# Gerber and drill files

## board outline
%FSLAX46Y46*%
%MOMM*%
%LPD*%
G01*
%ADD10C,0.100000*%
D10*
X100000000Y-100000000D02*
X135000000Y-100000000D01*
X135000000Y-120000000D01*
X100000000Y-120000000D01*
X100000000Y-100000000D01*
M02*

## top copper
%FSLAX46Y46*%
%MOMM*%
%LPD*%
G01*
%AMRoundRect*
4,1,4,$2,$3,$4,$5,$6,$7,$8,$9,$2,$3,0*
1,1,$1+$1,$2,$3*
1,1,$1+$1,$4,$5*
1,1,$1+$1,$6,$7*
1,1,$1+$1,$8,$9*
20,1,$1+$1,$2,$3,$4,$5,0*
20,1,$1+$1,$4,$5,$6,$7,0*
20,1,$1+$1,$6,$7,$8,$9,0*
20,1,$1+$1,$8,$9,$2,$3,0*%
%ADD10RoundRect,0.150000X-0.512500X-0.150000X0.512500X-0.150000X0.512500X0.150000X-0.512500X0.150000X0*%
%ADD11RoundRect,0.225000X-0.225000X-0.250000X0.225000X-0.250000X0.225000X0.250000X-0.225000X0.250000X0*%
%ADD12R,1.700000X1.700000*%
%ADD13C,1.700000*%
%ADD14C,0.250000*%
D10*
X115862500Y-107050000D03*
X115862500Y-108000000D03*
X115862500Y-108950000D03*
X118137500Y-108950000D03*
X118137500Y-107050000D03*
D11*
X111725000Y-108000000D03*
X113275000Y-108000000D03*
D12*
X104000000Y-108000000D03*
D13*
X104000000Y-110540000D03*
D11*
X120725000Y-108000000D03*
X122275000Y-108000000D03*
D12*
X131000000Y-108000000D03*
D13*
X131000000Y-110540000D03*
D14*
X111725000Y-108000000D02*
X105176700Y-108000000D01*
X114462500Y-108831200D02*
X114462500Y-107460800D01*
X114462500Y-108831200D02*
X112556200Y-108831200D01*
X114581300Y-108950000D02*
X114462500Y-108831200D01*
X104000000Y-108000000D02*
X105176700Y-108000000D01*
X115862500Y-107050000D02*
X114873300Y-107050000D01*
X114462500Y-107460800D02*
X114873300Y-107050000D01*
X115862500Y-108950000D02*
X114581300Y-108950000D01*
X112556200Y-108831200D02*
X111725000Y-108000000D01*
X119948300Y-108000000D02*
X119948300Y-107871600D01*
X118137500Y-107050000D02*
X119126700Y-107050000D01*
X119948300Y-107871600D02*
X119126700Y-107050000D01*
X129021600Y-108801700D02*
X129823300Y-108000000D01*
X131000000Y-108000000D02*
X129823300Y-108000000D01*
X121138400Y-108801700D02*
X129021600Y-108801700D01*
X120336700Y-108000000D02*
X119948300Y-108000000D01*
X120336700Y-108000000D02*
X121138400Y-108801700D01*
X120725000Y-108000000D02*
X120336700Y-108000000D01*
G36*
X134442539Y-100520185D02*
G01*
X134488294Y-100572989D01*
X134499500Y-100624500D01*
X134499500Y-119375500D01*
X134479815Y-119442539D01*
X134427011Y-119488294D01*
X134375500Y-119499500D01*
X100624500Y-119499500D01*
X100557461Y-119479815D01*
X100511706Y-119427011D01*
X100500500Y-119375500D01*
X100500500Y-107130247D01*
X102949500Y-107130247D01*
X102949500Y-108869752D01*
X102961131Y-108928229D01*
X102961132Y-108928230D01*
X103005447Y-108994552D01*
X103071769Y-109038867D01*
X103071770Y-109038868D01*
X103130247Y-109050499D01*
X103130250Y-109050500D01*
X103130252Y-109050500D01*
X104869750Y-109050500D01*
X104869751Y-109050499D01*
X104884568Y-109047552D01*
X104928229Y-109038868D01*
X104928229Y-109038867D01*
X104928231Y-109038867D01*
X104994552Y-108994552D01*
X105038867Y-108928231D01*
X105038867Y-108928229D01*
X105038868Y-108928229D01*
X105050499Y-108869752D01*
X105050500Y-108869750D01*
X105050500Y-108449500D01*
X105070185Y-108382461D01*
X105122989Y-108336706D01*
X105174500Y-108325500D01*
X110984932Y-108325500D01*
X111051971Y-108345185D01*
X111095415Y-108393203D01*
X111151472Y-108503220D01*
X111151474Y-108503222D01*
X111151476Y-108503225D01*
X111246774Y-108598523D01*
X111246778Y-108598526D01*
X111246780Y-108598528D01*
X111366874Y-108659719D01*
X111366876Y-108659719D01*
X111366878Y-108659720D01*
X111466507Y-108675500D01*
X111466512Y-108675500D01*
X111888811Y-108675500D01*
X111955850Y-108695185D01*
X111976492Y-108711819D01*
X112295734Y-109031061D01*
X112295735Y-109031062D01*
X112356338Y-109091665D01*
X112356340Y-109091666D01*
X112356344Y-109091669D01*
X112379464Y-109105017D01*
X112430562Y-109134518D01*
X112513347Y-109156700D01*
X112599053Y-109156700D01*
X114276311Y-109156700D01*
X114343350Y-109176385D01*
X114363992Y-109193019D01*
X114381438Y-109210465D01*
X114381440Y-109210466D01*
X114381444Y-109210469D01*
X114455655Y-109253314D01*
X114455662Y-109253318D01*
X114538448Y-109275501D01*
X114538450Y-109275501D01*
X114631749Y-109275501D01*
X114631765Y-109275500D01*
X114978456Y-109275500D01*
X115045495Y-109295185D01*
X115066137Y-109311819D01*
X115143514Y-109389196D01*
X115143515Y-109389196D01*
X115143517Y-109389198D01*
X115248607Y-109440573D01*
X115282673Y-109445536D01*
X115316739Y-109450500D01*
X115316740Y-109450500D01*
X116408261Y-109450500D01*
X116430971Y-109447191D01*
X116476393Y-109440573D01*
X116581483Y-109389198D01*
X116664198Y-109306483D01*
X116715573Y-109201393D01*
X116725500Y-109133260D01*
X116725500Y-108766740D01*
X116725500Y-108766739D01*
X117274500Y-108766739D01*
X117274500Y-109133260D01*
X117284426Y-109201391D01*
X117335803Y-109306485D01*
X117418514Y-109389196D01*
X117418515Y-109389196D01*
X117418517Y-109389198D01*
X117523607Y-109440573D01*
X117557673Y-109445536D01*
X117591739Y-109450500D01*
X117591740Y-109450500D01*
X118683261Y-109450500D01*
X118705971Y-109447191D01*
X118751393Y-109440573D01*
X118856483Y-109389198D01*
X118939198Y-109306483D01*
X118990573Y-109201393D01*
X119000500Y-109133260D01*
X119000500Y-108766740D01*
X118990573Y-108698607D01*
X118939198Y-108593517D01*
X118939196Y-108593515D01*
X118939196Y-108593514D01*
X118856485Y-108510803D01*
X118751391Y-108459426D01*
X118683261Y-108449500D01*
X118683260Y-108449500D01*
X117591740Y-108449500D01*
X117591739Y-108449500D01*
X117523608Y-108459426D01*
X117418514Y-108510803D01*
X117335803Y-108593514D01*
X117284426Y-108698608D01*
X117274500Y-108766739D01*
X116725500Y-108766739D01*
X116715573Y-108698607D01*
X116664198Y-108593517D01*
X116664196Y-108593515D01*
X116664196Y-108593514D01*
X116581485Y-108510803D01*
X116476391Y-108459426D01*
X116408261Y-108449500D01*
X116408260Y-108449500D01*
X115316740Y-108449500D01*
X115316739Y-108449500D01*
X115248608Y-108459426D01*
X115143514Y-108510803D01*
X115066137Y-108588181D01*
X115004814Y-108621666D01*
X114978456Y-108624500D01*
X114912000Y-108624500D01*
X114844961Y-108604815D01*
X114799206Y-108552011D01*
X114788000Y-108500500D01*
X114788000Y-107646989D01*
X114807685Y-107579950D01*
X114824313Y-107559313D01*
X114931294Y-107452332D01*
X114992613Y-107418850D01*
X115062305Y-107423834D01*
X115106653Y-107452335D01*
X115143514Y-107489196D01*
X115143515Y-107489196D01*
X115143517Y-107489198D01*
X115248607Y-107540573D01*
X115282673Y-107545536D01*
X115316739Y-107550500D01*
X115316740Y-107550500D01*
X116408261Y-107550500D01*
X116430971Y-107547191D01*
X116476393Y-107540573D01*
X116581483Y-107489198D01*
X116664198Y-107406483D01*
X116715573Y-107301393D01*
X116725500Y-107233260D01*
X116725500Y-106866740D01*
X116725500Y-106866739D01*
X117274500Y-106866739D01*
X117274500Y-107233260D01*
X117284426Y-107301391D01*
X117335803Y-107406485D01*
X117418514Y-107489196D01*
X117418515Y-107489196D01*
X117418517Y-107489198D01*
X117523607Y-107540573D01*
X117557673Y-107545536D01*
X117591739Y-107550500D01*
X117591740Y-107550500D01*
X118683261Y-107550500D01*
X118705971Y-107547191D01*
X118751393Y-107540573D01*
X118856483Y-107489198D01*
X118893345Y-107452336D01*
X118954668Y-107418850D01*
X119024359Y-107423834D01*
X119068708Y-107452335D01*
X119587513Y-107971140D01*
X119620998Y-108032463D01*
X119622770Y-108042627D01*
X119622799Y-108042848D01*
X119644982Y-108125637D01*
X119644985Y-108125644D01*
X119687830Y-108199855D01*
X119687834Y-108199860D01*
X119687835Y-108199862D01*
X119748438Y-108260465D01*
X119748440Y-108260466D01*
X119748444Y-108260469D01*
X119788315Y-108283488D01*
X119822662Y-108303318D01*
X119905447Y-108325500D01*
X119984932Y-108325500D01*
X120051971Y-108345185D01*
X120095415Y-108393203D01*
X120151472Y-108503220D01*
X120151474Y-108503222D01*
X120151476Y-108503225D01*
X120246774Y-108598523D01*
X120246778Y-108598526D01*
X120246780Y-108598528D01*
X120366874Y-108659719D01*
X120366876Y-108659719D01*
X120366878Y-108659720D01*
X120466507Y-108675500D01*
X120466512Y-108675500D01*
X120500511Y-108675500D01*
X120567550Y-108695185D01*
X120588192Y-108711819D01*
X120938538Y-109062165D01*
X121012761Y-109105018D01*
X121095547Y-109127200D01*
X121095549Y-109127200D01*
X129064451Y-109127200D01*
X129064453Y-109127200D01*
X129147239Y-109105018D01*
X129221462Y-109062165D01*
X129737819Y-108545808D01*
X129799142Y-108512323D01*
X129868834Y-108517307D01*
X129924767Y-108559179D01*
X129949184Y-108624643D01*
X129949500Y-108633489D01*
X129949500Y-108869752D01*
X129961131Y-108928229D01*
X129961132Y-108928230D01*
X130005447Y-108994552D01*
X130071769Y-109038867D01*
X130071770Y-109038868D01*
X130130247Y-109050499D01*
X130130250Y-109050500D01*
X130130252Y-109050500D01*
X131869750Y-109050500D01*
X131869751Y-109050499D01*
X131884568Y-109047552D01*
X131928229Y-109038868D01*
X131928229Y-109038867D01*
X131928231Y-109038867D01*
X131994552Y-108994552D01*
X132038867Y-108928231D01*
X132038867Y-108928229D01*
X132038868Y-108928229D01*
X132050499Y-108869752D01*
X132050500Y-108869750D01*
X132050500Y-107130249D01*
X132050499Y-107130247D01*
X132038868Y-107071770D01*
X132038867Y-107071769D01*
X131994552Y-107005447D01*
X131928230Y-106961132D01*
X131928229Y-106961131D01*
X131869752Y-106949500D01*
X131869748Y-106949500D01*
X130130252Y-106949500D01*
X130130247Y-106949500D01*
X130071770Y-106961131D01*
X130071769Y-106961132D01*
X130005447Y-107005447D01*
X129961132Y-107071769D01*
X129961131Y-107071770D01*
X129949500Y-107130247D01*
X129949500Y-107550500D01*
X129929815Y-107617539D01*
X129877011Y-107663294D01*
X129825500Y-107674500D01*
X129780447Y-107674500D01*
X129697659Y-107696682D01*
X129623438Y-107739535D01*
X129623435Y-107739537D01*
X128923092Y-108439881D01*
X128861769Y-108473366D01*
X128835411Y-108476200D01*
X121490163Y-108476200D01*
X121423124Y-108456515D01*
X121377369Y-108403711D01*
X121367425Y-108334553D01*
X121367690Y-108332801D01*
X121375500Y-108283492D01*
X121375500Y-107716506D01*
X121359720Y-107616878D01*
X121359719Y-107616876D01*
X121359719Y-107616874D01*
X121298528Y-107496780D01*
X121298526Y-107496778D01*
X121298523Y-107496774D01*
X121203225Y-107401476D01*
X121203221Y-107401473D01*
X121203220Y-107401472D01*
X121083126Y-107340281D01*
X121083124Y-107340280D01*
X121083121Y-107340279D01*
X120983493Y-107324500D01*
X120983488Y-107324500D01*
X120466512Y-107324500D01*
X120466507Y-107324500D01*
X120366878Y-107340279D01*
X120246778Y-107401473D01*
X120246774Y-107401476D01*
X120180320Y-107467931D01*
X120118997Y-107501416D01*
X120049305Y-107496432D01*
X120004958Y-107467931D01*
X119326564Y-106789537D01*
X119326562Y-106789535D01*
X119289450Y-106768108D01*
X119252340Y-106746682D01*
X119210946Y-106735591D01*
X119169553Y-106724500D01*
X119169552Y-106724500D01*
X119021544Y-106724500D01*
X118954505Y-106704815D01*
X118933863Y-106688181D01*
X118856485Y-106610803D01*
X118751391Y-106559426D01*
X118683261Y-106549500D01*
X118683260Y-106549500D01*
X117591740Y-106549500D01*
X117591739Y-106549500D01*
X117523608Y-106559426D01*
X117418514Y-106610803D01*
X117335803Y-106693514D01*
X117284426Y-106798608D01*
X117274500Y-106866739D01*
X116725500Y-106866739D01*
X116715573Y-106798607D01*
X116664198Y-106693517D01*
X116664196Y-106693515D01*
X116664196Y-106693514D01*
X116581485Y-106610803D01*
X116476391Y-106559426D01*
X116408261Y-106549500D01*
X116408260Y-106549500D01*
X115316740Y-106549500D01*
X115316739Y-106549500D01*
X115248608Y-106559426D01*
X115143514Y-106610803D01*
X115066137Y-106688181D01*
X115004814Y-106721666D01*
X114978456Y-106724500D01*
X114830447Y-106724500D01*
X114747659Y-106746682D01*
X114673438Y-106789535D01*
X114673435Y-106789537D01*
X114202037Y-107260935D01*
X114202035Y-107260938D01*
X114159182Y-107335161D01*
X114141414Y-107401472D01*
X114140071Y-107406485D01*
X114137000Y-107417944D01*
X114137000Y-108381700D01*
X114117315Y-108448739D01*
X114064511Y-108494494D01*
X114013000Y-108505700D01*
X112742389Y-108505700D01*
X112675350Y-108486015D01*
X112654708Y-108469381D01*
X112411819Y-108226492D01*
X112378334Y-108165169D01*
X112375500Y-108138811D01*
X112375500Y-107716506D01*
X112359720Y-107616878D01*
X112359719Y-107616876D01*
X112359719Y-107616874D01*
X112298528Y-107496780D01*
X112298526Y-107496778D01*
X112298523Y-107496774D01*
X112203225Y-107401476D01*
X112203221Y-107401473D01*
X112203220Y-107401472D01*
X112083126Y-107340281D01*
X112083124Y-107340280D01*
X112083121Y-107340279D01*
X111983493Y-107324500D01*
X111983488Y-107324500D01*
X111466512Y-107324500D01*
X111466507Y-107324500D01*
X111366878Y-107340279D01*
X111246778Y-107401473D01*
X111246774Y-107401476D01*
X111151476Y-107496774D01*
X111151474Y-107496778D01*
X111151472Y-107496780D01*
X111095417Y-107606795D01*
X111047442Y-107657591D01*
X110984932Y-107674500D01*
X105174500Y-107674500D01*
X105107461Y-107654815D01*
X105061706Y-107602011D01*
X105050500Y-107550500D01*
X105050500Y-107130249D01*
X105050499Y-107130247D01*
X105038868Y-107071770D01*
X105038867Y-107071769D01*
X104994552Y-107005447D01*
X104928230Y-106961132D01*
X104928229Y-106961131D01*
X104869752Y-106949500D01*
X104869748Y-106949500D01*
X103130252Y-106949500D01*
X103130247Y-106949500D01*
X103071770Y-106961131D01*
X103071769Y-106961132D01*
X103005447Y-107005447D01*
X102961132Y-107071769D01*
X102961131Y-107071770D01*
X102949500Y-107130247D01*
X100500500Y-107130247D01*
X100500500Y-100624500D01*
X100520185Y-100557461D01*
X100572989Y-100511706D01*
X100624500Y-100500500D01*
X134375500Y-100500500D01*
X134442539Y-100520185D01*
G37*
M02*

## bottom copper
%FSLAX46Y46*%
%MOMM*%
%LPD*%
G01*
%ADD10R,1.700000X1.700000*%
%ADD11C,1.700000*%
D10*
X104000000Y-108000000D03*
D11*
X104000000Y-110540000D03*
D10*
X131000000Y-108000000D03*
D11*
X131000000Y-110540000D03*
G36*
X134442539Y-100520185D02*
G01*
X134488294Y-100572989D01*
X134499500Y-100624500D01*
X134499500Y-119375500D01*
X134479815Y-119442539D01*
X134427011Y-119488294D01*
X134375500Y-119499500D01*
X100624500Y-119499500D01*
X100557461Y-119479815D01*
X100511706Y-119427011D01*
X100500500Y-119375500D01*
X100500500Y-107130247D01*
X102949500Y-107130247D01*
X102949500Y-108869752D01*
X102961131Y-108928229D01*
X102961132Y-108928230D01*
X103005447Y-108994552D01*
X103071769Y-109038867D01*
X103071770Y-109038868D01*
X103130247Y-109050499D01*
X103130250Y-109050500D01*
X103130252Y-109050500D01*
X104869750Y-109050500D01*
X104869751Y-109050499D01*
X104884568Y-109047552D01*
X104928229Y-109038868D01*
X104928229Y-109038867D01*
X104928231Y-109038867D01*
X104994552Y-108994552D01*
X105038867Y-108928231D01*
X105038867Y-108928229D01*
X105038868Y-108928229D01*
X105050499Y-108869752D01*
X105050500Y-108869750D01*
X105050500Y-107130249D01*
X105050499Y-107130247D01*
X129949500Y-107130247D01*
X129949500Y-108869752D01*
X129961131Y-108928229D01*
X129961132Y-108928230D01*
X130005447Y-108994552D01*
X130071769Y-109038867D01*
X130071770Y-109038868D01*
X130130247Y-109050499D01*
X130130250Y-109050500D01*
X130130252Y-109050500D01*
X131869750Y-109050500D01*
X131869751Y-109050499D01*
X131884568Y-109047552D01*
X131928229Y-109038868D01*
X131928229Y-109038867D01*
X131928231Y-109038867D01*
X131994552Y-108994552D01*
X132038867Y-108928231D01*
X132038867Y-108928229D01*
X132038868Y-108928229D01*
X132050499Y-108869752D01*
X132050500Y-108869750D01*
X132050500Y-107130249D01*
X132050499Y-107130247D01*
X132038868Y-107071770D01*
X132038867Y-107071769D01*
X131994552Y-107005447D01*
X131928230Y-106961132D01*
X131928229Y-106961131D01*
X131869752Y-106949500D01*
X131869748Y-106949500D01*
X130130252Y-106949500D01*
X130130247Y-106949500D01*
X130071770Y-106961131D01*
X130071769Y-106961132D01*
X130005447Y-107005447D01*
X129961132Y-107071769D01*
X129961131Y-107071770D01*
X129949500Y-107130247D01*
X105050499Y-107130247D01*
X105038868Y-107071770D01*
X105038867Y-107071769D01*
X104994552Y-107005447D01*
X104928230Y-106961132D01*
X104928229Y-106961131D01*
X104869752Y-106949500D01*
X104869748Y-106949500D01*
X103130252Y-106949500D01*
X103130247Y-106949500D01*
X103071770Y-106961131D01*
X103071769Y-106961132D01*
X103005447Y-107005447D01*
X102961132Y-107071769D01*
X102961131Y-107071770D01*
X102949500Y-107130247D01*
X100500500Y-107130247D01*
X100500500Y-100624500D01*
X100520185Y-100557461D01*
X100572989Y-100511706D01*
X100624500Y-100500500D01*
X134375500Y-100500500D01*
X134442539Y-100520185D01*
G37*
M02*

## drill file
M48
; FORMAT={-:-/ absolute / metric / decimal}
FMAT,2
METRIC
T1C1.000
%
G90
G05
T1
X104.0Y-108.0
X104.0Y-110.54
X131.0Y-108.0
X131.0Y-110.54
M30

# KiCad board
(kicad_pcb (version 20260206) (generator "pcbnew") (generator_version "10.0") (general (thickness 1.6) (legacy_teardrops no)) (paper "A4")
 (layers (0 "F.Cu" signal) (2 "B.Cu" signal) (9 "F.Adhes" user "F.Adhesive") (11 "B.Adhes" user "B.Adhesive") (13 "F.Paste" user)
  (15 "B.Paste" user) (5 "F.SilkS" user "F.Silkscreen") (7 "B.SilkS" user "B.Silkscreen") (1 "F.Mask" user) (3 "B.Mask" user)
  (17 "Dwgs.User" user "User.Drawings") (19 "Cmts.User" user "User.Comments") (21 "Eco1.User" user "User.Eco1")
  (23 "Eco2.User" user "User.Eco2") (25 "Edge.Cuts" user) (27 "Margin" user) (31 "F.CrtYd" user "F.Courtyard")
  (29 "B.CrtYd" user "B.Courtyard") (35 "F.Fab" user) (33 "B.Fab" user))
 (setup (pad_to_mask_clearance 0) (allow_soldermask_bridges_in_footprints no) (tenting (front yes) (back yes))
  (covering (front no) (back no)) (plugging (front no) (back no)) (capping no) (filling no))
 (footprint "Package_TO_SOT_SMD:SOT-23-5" (layer "F.Cu") (at 117 108)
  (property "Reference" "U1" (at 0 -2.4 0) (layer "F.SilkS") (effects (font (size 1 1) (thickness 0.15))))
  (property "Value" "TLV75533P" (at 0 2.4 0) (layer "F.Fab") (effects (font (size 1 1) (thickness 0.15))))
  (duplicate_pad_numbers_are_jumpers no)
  (pad "1" smd roundrect (at -1.1375 -0.95) (size 1.325 0.6) (layers "F.Cu" "F.Mask" "F.Paste") (roundrect_rratio 0.25) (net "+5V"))
  (pad "2" smd roundrect (at -1.1375 0) (size 1.325 0.6) (layers "F.Cu" "F.Mask" "F.Paste") (roundrect_rratio 0.25) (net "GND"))
  (pad "3" smd roundrect (at -1.1375 0.95) (size 1.325 0.6) (layers "F.Cu" "F.Mask" "F.Paste") (roundrect_rratio 0.25) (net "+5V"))
  (pad "4" smd roundrect (at 1.1375 0.95) (size 1.325 0.6) (layers "F.Cu" "F.Mask" "F.Paste") (roundrect_rratio 0.25)
   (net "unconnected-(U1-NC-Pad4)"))
  (pad "5" smd roundrect (at 1.1375 -0.95) (size 1.325 0.6) (layers "F.Cu" "F.Mask" "F.Paste") (roundrect_rratio 0.25) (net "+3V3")))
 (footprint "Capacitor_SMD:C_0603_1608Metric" (layer "F.Cu") (at 112.5 108)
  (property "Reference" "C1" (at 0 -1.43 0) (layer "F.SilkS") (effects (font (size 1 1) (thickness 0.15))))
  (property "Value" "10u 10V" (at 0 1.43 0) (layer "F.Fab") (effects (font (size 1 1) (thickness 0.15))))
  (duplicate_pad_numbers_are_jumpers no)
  (pad "1" smd roundrect (at -0.775 0) (size 0.9 0.95) (layers "F.Cu" "F.Mask" "F.Paste") (roundrect_rratio 0.25) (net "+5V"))
  (pad "2" smd roundrect (at 0.775 0) (size 0.9 0.95) (layers "F.Cu" "F.Mask" "F.Paste") (roundrect_rratio 0.25) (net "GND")))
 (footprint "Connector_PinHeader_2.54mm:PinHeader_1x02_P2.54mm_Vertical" (layer "F.Cu") (at 104 108)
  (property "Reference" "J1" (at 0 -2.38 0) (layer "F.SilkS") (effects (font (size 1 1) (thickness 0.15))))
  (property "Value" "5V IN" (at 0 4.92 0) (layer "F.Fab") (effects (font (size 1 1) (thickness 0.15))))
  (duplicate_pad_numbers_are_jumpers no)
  (pad "1" thru_hole rect (at 0 0) (size 1.7 1.7) (drill 1) (layers "*.Cu" "*.Mask") (remove_unused_layers no) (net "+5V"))
  (pad "2" thru_hole circle (at 0 2.54) (size 1.7 1.7) (drill 1) (layers "*.Cu" "*.Mask") (remove_unused_layers no) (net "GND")))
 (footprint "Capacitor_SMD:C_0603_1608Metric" (layer "F.Cu") (at 121.5 108)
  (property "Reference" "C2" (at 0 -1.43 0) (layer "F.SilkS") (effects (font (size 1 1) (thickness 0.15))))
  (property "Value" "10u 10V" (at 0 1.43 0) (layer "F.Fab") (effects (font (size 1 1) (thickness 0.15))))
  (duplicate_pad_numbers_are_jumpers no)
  (pad "1" smd roundrect (at -0.775 0) (size 0.9 0.95) (layers "F.Cu" "F.Mask" "F.Paste") (roundrect_rratio 0.25) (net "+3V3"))
  (pad "2" smd roundrect (at 0.775 0) (size 0.9 0.95) (layers "F.Cu" "F.Mask" "F.Paste") (roundrect_rratio 0.25) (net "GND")))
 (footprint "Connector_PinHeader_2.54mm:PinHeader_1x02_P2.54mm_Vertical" (layer "F.Cu") (at 131 108)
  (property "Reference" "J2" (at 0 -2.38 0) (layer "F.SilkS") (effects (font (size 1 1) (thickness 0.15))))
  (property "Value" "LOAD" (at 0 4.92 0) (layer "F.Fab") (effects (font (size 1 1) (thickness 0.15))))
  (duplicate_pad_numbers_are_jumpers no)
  (pad "1" thru_hole rect (at 0 0) (size 1.7 1.7) (drill 1) (layers "*.Cu" "*.Mask") (remove_unused_layers no) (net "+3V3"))
  (pad "2" thru_hole circle (at 0 2.54) (size 1.7 1.7) (drill 1) (layers "*.Cu" "*.Mask") (remove_unused_layers no) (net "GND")))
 (gr_rect (start 100 100) (end 135 120) (stroke (width 0.1) (type default)) (fill no) (layer "Edge.Cuts"))
 (segment (start 111.725 108) (end 105.1767 108) (width 0.25) (layer "F.Cu") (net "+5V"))
 (segment (start 114.4625 108.8312) (end 114.4625 107.4608) (width 0.25) (layer "F.Cu") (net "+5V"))
 (segment (start 114.4625 108.8312) (end 112.5562 108.8312) (width 0.25) (layer "F.Cu") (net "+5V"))
 (segment (start 114.5813 108.95) (end 114.4625 108.8312) (width 0.25) (layer "F.Cu") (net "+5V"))
 (segment (start 104 108) (end 105.1767 108) (width 0.25) (layer "F.Cu") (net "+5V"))
 (segment (start 115.8625 107.05) (end 114.8733 107.05) (width 0.25) (layer "F.Cu") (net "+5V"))
 (segment (start 114.4625 107.4608) (end 114.8733 107.05) (width 0.25) (layer "F.Cu") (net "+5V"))
 (segment (start 115.8625 108.95) (end 114.5813 108.95) (width 0.25) (layer "F.Cu") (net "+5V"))
 (segment (start 112.5562 108.8312) (end 111.725 108) (width 0.25) (layer "F.Cu") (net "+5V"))
 (segment (start 119.9483 108) (end 119.9483 107.8716) (width 0.25) (layer "F.Cu") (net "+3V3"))
 (segment (start 118.1375 107.05) (end 119.1267 107.05) (width 0.25) (layer "F.Cu") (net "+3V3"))
 (segment (start 119.9483 107.8716) (end 119.1267 107.05) (width 0.25) (layer "F.Cu") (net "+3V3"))
 (segment (start 129.0216 108.8017) (end 129.8233 108) (width 0.25) (layer "F.Cu") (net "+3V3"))
 (segment (start 131 108) (end 129.8233 108) (width 0.25) (layer "F.Cu") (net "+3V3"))
 (segment (start 121.1384 108.8017) (end 129.0216 108.8017) (width 0.25) (layer "F.Cu") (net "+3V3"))
 (segment (start 120.3367 108) (end 119.9483 108) (width 0.25) (layer "F.Cu") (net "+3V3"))
 (segment (start 120.3367 108) (end 121.1384 108.8017) (width 0.25) (layer "F.Cu") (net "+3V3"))
 (segment (start 120.725 108) (end 120.3367 108) (width 0.25) (layer "F.Cu") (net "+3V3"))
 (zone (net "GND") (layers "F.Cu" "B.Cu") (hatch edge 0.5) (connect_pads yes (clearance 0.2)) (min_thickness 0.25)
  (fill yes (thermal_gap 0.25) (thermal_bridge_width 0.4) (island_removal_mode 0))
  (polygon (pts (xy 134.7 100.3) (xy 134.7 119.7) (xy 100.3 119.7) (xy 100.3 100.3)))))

